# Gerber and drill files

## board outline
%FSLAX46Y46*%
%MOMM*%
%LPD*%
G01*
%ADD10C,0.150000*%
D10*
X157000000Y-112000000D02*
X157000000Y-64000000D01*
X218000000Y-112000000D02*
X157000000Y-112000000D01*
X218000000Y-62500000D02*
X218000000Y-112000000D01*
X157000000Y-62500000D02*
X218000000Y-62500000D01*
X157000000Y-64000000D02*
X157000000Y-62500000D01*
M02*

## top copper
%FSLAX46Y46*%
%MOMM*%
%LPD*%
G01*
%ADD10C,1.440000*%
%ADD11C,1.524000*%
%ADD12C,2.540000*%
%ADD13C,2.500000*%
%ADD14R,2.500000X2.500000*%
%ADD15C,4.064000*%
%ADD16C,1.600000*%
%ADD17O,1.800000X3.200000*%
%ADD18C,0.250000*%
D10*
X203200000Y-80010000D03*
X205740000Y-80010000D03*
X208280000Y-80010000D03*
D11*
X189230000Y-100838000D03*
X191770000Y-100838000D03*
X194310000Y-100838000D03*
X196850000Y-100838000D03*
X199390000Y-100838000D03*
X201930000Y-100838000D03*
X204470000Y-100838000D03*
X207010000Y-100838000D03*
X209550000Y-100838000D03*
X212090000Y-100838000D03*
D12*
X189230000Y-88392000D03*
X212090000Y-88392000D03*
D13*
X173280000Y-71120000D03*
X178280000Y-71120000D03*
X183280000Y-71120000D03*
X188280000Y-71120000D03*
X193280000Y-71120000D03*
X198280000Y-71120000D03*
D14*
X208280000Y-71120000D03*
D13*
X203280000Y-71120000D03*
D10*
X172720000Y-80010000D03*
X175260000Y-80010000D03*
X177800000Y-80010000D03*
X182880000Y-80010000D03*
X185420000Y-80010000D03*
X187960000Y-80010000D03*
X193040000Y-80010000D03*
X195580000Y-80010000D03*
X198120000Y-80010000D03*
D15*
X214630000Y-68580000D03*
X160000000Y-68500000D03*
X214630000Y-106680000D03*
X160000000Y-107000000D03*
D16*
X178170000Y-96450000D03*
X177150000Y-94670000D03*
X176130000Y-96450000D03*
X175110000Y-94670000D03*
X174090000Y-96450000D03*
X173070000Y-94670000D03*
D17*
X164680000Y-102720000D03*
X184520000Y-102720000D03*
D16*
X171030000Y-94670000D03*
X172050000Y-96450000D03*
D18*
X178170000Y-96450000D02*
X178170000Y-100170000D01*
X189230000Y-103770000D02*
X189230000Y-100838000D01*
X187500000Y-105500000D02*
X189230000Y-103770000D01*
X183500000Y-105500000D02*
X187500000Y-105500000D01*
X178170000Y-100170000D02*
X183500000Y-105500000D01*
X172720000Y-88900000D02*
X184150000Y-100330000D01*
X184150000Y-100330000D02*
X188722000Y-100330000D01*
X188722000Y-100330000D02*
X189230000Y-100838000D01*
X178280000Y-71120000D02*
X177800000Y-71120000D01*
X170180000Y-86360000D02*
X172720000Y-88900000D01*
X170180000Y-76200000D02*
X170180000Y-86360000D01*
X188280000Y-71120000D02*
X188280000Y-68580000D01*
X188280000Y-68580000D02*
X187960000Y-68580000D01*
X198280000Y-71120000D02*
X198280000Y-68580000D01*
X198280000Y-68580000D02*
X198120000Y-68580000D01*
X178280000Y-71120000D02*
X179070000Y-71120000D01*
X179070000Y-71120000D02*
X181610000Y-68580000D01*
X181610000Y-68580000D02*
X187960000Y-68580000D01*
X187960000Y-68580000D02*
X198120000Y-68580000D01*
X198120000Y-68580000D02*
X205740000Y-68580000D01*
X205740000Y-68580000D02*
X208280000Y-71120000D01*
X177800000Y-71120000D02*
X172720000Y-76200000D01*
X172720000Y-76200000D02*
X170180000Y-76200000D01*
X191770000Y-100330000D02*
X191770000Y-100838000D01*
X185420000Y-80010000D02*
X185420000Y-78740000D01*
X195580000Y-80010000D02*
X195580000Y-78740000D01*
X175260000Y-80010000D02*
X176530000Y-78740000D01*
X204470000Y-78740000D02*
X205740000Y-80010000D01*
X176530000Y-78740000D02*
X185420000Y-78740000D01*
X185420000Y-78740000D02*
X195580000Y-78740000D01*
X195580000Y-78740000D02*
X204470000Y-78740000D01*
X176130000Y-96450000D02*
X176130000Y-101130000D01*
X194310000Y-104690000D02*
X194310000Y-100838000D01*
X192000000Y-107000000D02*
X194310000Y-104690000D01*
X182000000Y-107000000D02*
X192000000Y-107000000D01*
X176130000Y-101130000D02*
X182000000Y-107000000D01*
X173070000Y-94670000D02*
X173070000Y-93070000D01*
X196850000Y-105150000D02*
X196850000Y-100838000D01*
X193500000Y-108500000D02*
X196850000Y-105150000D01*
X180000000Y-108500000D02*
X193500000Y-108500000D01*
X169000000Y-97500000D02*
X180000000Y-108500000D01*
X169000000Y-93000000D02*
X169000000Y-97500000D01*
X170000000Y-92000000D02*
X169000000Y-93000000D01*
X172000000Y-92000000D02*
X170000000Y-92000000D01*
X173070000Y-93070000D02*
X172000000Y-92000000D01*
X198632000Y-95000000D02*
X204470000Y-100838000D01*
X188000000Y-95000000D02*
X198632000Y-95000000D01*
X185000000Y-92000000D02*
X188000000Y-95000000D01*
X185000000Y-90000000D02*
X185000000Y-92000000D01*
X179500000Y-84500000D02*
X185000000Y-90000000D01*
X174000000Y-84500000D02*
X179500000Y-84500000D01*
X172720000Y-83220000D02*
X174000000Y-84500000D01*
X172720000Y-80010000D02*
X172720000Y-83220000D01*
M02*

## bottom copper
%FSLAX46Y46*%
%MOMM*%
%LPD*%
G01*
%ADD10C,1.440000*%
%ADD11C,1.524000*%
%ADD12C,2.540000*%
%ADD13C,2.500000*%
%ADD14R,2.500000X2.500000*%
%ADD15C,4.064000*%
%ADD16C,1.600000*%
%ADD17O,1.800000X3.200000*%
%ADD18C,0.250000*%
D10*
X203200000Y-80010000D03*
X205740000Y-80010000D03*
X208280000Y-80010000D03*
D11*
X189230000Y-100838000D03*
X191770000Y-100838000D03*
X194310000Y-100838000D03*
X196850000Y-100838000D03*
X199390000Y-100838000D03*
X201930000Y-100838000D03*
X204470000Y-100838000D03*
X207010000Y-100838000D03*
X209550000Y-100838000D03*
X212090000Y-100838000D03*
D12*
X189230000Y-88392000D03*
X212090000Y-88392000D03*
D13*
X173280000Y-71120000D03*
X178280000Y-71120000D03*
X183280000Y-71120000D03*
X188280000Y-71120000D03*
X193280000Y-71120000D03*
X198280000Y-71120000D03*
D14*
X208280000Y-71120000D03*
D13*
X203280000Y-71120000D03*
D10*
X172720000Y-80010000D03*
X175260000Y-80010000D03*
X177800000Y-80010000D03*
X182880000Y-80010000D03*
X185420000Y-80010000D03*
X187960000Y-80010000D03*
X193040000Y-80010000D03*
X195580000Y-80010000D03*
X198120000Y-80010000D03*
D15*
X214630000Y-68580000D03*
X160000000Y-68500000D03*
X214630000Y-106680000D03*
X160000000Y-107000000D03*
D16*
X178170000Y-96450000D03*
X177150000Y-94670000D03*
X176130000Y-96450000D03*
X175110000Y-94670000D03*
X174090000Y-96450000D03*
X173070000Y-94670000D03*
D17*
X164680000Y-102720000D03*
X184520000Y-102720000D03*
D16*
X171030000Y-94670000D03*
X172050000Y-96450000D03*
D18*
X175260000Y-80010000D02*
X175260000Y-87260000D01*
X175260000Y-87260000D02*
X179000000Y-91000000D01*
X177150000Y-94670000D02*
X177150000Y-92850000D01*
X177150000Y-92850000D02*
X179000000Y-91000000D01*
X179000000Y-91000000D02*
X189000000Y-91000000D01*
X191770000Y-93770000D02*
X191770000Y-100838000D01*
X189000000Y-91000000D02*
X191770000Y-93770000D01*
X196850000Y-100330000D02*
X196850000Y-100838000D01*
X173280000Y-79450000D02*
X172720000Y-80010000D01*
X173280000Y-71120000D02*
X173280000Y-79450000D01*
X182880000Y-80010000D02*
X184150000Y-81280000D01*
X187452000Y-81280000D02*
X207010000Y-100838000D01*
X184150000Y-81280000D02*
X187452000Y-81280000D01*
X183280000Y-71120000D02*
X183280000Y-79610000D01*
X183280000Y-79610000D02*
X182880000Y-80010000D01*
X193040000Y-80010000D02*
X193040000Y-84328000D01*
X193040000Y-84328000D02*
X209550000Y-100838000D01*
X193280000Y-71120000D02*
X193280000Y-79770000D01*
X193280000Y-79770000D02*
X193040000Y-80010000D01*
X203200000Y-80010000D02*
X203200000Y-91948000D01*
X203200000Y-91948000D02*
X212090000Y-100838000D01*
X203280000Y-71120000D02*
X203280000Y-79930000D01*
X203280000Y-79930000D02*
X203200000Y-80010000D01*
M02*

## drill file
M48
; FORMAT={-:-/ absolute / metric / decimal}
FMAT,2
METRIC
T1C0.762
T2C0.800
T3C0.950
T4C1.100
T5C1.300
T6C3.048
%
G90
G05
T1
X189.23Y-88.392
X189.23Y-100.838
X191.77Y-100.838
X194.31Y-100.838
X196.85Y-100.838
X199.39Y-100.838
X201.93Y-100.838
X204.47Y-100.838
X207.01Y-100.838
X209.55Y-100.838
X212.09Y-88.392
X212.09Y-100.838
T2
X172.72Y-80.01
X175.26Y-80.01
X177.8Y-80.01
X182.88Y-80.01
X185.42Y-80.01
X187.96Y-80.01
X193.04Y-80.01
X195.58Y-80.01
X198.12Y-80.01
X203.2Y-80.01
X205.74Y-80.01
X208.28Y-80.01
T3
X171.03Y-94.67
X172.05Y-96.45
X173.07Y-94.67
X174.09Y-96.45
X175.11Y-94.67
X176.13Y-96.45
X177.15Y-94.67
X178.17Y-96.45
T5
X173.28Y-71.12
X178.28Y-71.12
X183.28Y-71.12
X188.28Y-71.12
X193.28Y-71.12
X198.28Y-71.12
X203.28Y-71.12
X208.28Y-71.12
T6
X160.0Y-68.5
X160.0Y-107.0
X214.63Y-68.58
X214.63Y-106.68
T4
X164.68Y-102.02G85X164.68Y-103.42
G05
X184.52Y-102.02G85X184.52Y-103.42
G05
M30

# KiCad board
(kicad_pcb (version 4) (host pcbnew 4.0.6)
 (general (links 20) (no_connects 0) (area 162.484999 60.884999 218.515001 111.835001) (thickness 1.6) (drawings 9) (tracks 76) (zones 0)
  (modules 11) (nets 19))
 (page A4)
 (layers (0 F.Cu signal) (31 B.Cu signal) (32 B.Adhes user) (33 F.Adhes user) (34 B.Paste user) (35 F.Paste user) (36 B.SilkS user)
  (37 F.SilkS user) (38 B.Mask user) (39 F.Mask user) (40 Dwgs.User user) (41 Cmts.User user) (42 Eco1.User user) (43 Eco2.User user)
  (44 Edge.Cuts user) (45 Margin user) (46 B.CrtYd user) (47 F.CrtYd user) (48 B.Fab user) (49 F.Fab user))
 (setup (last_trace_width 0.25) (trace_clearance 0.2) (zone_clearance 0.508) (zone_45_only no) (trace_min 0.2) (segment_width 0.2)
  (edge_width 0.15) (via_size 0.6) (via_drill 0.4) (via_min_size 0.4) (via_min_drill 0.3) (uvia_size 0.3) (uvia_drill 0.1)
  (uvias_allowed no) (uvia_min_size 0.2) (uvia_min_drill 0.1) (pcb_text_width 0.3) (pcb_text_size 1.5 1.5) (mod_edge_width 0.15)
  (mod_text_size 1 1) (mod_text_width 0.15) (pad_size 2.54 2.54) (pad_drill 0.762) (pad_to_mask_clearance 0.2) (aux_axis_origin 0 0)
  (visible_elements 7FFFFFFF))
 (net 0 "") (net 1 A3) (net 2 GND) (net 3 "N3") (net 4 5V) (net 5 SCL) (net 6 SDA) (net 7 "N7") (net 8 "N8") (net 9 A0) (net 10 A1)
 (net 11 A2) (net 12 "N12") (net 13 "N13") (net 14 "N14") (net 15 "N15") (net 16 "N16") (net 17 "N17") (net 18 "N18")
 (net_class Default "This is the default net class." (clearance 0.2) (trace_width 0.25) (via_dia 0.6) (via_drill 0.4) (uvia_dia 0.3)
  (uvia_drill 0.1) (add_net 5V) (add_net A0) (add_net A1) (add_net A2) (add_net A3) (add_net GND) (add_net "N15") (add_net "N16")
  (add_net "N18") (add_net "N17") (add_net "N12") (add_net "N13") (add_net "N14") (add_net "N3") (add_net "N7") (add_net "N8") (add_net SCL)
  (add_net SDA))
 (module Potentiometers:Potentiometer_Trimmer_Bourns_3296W (layer F.Cu) (at 203.2 80.01 180)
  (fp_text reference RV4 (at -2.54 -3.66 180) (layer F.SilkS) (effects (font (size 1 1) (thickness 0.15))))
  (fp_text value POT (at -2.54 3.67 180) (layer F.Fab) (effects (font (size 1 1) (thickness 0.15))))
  (pad 1 thru_hole circle (at 0 0 180) (size 1.44 1.44) (drill 0.8) (layers *.Cu *.Mask) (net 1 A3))
  (pad 2 thru_hole circle (at -2.54 0 180) (size 1.44 1.44) (drill 0.8) (layers *.Cu *.Mask) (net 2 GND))
  (pad 3 thru_hole circle (at -5.08 0 180) (size 1.44 1.44) (drill 0.8) (layers *.Cu *.Mask) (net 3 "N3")))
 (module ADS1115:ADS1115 (layer F.Cu) (at 201.93 102.87 90)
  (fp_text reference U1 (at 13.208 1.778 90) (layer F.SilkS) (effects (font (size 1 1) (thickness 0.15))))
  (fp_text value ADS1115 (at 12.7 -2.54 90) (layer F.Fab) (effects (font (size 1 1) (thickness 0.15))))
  (pad 1 thru_hole circle (at 2.032 -12.7 90) (size 1.524 1.524) (drill 0.762) (layers *.Cu *.Mask) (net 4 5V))
  (pad 2 thru_hole circle (at 2.032 -10.16 90) (size 1.524 1.524) (drill 0.762) (layers *.Cu *.Mask) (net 2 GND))
  (pad 3 thru_hole circle (at 2.032 -7.62 90) (size 1.524 1.524) (drill 0.762) (layers *.Cu *.Mask) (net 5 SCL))
  (pad 4 thru_hole circle (at 2.032 -5.08 90) (size 1.524 1.524) (drill 0.762) (layers *.Cu *.Mask) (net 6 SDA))
  (pad 5 thru_hole circle (at 2.032 -2.54 90) (size 1.524 1.524) (drill 0.762) (layers *.Cu *.Mask) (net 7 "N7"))
  (pad 6 thru_hole circle (at 2.032 0 90) (size 1.524 1.524) (drill 0.762) (layers *.Cu *.Mask) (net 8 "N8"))
  (pad 7 thru_hole circle (at 2.032 2.54 90) (size 1.524 1.524) (drill 0.762) (layers *.Cu *.Mask) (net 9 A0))
  (pad 8 thru_hole circle (at 2.032 5.08 90) (size 1.524 1.524) (drill 0.762) (layers *.Cu *.Mask) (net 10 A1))
  (pad 9 thru_hole circle (at 2.032 7.62 90) (size 1.524 1.524) (drill 0.762) (layers *.Cu *.Mask) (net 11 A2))
  (pad 10 thru_hole circle (at 2.032 10.16 90) (size 1.524 1.524) (drill 0.762) (layers *.Cu *.Mask) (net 1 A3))
  (pad "" thru_hole circle (at 14.478 -12.7 90) (size 2.54 2.54) (drill 0.762) (layers *.Cu *.Mask))
  (pad "" thru_hole circle (at 14.478 10.16 90) (size 2.54 2.54) (drill 0.762) (layers *.Cu *.Mask)))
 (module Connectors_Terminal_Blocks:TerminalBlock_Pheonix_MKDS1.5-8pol (layer F.Cu) (at 208.28 71.12 180)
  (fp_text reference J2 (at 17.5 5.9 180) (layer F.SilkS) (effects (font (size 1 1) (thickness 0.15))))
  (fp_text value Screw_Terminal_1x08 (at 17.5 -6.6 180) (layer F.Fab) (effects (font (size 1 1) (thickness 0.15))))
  (pad 8 thru_hole circle (at 35 0 180) (size 2.5 2.5) (drill 1.3) (layers *.Cu *.Mask) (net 9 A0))
  (pad 7 thru_hole circle (at 30 0 180) (size 2.5 2.5) (drill 1.3) (layers *.Cu *.Mask) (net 4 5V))
  (pad 6 thru_hole circle (at 25 0 180) (size 2.5 2.5) (drill 1.3) (layers *.Cu *.Mask) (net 10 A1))
  (pad 5 thru_hole circle (at 20 0 180) (size 2.5 2.5) (drill 1.3) (layers *.Cu *.Mask) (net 4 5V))
  (pad 4 thru_hole circle (at 15 0 180) (size 2.5 2.5) (drill 1.3) (layers *.Cu *.Mask) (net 11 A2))
  (pad 3 thru_hole circle (at 10 0 180) (size 2.5 2.5) (drill 1.3) (layers *.Cu *.Mask) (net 4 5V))
  (pad 1 thru_hole rect (at 0 0 180) (size 2.5 2.5) (drill 1.3) (layers *.Cu *.Mask) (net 4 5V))
  (pad 2 thru_hole circle (at 5 0 180) (size 2.5 2.5) (drill 1.3) (layers *.Cu *.Mask) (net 1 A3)))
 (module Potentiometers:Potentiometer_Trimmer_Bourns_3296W (layer F.Cu) (at 172.72 80.01 180)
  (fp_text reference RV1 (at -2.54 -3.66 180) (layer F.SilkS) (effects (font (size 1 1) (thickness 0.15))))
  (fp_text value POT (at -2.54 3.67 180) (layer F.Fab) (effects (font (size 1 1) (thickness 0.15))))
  (pad 1 thru_hole circle (at 0 0 180) (size 1.44 1.44) (drill 0.8) (layers *.Cu *.Mask) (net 9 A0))
  (pad 2 thru_hole circle (at -2.54 0 180) (size 1.44 1.44) (drill 0.8) (layers *.Cu *.Mask) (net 2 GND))
  (pad 3 thru_hole circle (at -5.08 0 180) (size 1.44 1.44) (drill 0.8) (layers *.Cu *.Mask) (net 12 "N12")))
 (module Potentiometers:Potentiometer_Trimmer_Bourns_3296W (layer F.Cu) (at 182.88 80.01 180)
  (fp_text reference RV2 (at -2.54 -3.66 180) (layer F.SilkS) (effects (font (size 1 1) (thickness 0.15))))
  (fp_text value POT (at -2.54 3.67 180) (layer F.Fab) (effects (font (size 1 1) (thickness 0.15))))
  (pad 1 thru_hole circle (at 0 0 180) (size 1.44 1.44) (drill 0.8) (layers *.Cu *.Mask) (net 10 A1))
  (pad 2 thru_hole circle (at -2.54 0 180) (size 1.44 1.44) (drill 0.8) (layers *.Cu *.Mask) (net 2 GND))
  (pad 3 thru_hole circle (at -5.08 0 180) (size 1.44 1.44) (drill 0.8) (layers *.Cu *.Mask) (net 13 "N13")))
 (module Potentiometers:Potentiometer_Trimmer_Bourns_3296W (layer F.Cu) (at 193.04 80.01 180)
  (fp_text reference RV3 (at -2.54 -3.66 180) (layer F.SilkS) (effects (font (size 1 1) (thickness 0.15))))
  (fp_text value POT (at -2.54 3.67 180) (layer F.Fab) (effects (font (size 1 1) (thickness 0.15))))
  (pad 1 thru_hole circle (at 0 0 180) (size 1.44 1.44) (drill 0.8) (layers *.Cu *.Mask) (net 11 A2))
  (pad 2 thru_hole circle (at -2.54 0 180) (size 1.44 1.44) (drill 0.8) (layers *.Cu *.Mask) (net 2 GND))
  (pad 3 thru_hole circle (at -5.08 0 180) (size 1.44 1.44) (drill 0.8) (layers *.Cu *.Mask) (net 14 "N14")))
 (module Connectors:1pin (layer F.Cu) (at 214.63 68.58)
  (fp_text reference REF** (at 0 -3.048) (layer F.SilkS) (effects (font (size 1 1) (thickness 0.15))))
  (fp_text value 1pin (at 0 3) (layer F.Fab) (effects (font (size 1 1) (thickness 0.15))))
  (pad 1 thru_hole circle (at 0 0) (size 4.064 4.064) (drill 3.048) (layers *.Cu *.Mask)))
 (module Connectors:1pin (layer F.Cu) (at 160 68.5)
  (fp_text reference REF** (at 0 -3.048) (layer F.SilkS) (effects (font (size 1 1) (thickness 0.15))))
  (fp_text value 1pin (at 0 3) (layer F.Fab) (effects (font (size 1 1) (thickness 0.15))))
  (pad 1 thru_hole circle (at 0 0) (size 4.064 4.064) (drill 3.048) (layers *.Cu *.Mask)))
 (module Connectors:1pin (layer F.Cu) (at 214.63 106.68)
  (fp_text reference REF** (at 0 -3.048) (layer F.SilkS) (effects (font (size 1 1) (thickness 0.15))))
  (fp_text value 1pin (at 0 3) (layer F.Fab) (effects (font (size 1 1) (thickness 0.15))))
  (pad 1 thru_hole circle (at 0 0) (size 4.064 4.064) (drill 3.048) (layers *.Cu *.Mask)))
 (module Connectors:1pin (layer F.Cu) (at 160 107)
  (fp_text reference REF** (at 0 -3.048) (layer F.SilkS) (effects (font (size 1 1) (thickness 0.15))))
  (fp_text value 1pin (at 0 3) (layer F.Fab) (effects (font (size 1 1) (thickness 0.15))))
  (pad 1 thru_hole circle (at 0 0) (size 4.064 4.064) (drill 3.048) (layers *.Cu *.Mask)))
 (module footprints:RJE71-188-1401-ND (layer F.Cu) (at 166.5 91)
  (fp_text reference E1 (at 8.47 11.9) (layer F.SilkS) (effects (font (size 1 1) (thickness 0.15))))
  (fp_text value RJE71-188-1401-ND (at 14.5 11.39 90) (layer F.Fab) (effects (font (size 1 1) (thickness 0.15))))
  (pad 1 thru_hole circle (at 11.67 5.45) (size 1.6 1.6) (drill 0.95) (layers *.Cu *.Mask) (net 4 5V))
  (pad 2 thru_hole circle (at 10.65 3.67) (size 1.6 1.6) (drill 0.95) (layers *.Cu *.Mask) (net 2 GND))
  (pad 3 thru_hole circle (at 9.63 5.45) (size 1.6 1.6) (drill 0.95) (layers *.Cu *.Mask) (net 5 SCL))
  (pad 4 thru_hole circle (at 8.61 3.67) (size 1.6 1.6) (drill 0.95) (layers *.Cu *.Mask) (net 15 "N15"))
  (pad 5 thru_hole circle (at 7.59 5.45) (size 1.6 1.6) (drill 0.95) (layers *.Cu *.Mask) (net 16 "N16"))
  (pad 6 thru_hole circle (at 6.57 3.67) (size 1.6 1.6) (drill 0.95) (layers *.Cu *.Mask) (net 6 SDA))
  (pad "" thru_hole oval (at -1.82 11.72) (size 1.8 3.2) (drill oval 1.1 2.5) (layers *.Cu *.Mask))
  (pad "" thru_hole oval (at 18.02 11.72) (size 1.8 3.2) (drill oval 1.1 2.5) (layers *.Cu *.Mask))
  (pad 8 thru_hole circle (at 4.53 3.67) (size 1.6 1.6) (drill 0.95) (layers *.Cu *.Mask) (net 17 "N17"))
  (pad 7 thru_hole circle (at 5.55 5.45) (size 1.6 1.6) (drill 0.95) (layers *.Cu *.Mask) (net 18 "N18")))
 (gr_line (start 157 112) (end 157 64) (angle 90) (layer Edge.Cuts) (width 0.15))
 (gr_line (start 218 112) (end 157 112) (angle 90) (layer Edge.Cuts) (width 0.15))
 (gr_line (start 218 62.5) (end 218 112) (angle 90) (layer Edge.Cuts) (width 0.15))
 (gr_line (start 157 62.5) (end 218 62.5) (angle 90) (layer Edge.Cuts) (width 0.15))
 (gr_line (start 157 64) (end 157 62.5) (angle 90) (layer Edge.Cuts) (width 0.15))
 (segment (start 178.17 96.45) (end 178.17 100.17) (width 0.25) (layer F.Cu) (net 4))
 (segment (start 189.23 103.77) (end 189.23 100.838) (width 0.25) (layer F.Cu) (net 4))
 (segment (start 187.5 105.5) (end 189.23 103.77) (width 0.25) (layer F.Cu) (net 4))
 (segment (start 183.5 105.5) (end 187.5 105.5) (width 0.25) (layer F.Cu) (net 4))
 (segment (start 178.17 100.17) (end 183.5 105.5) (width 0.25) (layer F.Cu) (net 4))
 (segment (start 172.72 88.9) (end 184.15 100.33) (width 0.25) (layer F.Cu) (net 4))
 (segment (start 184.15 100.33) (end 188.722 100.33) (width 0.25) (layer F.Cu) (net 4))
 (segment (start 188.722 100.33) (end 189.23 100.838) (width 0.25) (layer F.Cu) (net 4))
 (segment (start 178.28 71.12) (end 177.8 71.12) (width 0.25) (layer F.Cu) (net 4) (status 30))
 (segment (start 170.18 86.36) (end 172.72 88.9) (width 0.25) (layer F.Cu) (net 4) (status 20))
 (segment (start 170.18 76.2) (end 170.18 86.36) (width 0.25) (layer F.Cu) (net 4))
 (segment (start 188.28 71.12) (end 188.28 68.58) (width 0.25) (layer F.Cu) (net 4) (status 10))
 (segment (start 188.28 68.58) (end 187.96 68.58) (width 0.25) (layer F.Cu) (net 4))
 (segment (start 198.28 71.12) (end 198.28 68.58) (width 0.25) (layer F.Cu) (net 4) (status 10))
 (segment (start 198.28 68.58) (end 198.12 68.58) (width 0.25) (layer F.Cu) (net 4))
 (segment (start 178.28 71.12) (end 179.07 71.12) (width 0.25) (layer F.Cu) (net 4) (status 30))
 (segment (start 179.07 71.12) (end 181.61 68.58) (width 0.25) (layer F.Cu) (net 4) (status 10))
 (segment (start 181.61 68.58) (end 187.96 68.58) (width 0.25) (layer F.Cu) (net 4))
 (segment (start 187.96 68.58) (end 198.12 68.58) (width 0.25) (layer F.Cu) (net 4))
 (segment (start 198.12 68.58) (end 205.74 68.58) (width 0.25) (layer F.Cu) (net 4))
 (segment (start 205.74 68.58) (end 208.28 71.12) (width 0.25) (layer F.Cu) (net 4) (status 20))
 (segment (start 177.8 71.12) (end 172.72 76.2) (width 0.25) (layer F.Cu) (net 4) (status 10))
 (segment (start 172.72 76.2) (end 170.18 76.2) (width 0.25) (layer F.Cu) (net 4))
 (segment (start 175.26 80.01) (end 175.26 87.26) (width 0.25) (layer B.Cu) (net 2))
 (segment (start 175.26 87.26) (end 179 91) (width 0.25) (layer B.Cu) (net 2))
 (segment (start 177.15 94.67) (end 177.15 92.85) (width 0.25) (layer B.Cu) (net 2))
 (segment (start 177.15 92.85) (end 179 91) (width 0.25) (layer B.Cu) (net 2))
 (segment (start 179 91) (end 189 91) (width 0.25) (layer B.Cu) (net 2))
 (segment (start 191.77 93.77) (end 191.77 100.838) (width 0.25) (layer B.Cu) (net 2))
 (segment (start 189 91) (end 191.77 93.77) (width 0.25) (layer B.Cu) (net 2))
 (segment (start 191.77 100.33) (end 191.77 100.838) (width 0.25) (layer F.Cu) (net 2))
 (segment (start 185.42 80.01) (end 185.42 78.74) (width 0.25) (layer F.Cu) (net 2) (status 10))
 (segment (start 195.58 80.01) (end 195.58 78.74) (width 0.25) (layer F.Cu) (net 2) (status 10))
 (segment (start 175.26 80.01) (end 176.53 78.74) (width 0.25) (layer F.Cu) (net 2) (status 10))
 (segment (start 204.47 78.74) (end 205.74 80.01) (width 0.25) (layer F.Cu) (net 2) (status 20))
 (segment (start 176.53 78.74) (end 185.42 78.74) (width 0.25) (layer F.Cu) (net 2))
 (segment (start 185.42 78.74) (end 195.58 78.74) (width 0.25) (layer F.Cu) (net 2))
 (segment (start 195.58 78.74) (end 204.47 78.74) (width 0.25) (layer F.Cu) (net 2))
 (segment (start 176.13 96.45) (end 176.13 101.13) (width 0.25) (layer F.Cu) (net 5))
 (segment (start 194.31 104.69) (end 194.31 100.838) (width 0.25) (layer F.Cu) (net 5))
 (segment (start 192 107) (end 194.31 104.69) (width 0.25) (layer F.Cu) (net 5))
 (segment (start 182 107) (end 192 107) (width 0.25) (layer F.Cu) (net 5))
 (segment (start 176.13 101.13) (end 182 107) (width 0.25) (layer F.Cu) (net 5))
 (segment (start 173.07 94.67) (end 173.07 93.07) (width 0.25) (layer F.Cu) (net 6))
 (segment (start 196.85 105.15) (end 196.85 100.838) (width 0.25) (layer F.Cu) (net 6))
 (segment (start 193.5 108.5) (end 196.85 105.15) (width 0.25) (layer F.Cu) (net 6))
 (segment (start 180 108.5) (end 193.5 108.5) (width 0.25) (layer F.Cu) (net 6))
 (segment (start 169 97.5) (end 180 108.5) (width 0.25) (layer F.Cu) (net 6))
 (segment (start 169 93) (end 169 97.5) (width 0.25) (layer F.Cu) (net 6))
 (segment (start 170 92) (end 169 93) (width 0.25) (layer F.Cu) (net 6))
 (segment (start 172 92) (end 170 92) (width 0.25) (layer F.Cu) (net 6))
 (segment (start 173.07 93.07) (end 172 92) (width 0.25) (layer F.Cu) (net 6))
 (segment (start 196.85 100.33) (end 196.85 100.838) (width 0.25) (layer B.Cu) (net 6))
 (segment (start 198.632 95) (end 204.47 100.838) (width 0.25) (layer F.Cu) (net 9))
 (segment (start 188 95) (end 198.632 95) (width 0.25) (layer F.Cu) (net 9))
 (segment (start 185 92) (end 188 95) (width 0.25) (layer F.Cu) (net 9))
 (segment (start 185 90) (end 185 92) (width 0.25) (layer F.Cu) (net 9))
 (segment (start 179.5 84.5) (end 185 90) (width 0.25) (layer F.Cu) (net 9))
 (segment (start 174 84.5) (end 179.5 84.5) (width 0.25) (layer F.Cu) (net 9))
 (segment (start 172.72 83.22) (end 174 84.5) (width 0.25) (layer F.Cu) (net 9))
 (segment (start 172.72 80.01) (end 172.72 83.22) (width 0.25) (layer F.Cu) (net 9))
 (segment (start 173.28 79.45) (end 172.72 80.01) (width 0.25) (layer B.Cu) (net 9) (status 20))
 (segment (start 173.28 71.12) (end 173.28 79.45) (width 0.25) (layer B.Cu) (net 9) (status 10))
 (segment (start 182.88 80.01) (end 184.15 81.28) (width 0.25) (layer B.Cu) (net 10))
 (segment (start 187.452 81.28) (end 207.01 100.838) (width 0.25) (layer B.Cu) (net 10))
 (segment (start 184.15 81.28) (end 187.452 81.28) (width 0.25) (layer B.Cu) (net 10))
 (segment (start 183.28 71.12) (end 183.28 79.61) (width 0.25) (layer B.Cu) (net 10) (status 30))
 (segment (start 183.28 79.61) (end 182.88 80.01) (width 0.25) (layer B.Cu) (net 10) (status 30))
 (segment (start 193.04 80.01) (end 193.04 84.328) (width 0.25) (layer B.Cu) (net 11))
 (segment (start 193.04 84.328) (end 209.55 100.838) (width 0.25) (layer B.Cu) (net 11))
 (segment (start 193.28 71.12) (end 193.28 79.77) (width 0.25) (layer B.Cu) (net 11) (status 30))
 (segment (start 193.28 79.77) (end 193.04 80.01) (width 0.25) (layer B.Cu) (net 11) (status 30))
 (segment (start 203.2 80.01) (end 203.2 91.948) (width 0.25) (layer B.Cu) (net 1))
 (segment (start 203.2 91.948) (end 212.09 100.838) (width 0.25) (layer B.Cu) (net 1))
 (segment (start 203.28 71.12) (end 203.28 79.93) (width 0.25) (layer B.Cu) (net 1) (status 30))
 (segment (start 203.28 79.93) (end 203.2 80.01) (width 0.25) (layer B.Cu) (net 1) (status 30)))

